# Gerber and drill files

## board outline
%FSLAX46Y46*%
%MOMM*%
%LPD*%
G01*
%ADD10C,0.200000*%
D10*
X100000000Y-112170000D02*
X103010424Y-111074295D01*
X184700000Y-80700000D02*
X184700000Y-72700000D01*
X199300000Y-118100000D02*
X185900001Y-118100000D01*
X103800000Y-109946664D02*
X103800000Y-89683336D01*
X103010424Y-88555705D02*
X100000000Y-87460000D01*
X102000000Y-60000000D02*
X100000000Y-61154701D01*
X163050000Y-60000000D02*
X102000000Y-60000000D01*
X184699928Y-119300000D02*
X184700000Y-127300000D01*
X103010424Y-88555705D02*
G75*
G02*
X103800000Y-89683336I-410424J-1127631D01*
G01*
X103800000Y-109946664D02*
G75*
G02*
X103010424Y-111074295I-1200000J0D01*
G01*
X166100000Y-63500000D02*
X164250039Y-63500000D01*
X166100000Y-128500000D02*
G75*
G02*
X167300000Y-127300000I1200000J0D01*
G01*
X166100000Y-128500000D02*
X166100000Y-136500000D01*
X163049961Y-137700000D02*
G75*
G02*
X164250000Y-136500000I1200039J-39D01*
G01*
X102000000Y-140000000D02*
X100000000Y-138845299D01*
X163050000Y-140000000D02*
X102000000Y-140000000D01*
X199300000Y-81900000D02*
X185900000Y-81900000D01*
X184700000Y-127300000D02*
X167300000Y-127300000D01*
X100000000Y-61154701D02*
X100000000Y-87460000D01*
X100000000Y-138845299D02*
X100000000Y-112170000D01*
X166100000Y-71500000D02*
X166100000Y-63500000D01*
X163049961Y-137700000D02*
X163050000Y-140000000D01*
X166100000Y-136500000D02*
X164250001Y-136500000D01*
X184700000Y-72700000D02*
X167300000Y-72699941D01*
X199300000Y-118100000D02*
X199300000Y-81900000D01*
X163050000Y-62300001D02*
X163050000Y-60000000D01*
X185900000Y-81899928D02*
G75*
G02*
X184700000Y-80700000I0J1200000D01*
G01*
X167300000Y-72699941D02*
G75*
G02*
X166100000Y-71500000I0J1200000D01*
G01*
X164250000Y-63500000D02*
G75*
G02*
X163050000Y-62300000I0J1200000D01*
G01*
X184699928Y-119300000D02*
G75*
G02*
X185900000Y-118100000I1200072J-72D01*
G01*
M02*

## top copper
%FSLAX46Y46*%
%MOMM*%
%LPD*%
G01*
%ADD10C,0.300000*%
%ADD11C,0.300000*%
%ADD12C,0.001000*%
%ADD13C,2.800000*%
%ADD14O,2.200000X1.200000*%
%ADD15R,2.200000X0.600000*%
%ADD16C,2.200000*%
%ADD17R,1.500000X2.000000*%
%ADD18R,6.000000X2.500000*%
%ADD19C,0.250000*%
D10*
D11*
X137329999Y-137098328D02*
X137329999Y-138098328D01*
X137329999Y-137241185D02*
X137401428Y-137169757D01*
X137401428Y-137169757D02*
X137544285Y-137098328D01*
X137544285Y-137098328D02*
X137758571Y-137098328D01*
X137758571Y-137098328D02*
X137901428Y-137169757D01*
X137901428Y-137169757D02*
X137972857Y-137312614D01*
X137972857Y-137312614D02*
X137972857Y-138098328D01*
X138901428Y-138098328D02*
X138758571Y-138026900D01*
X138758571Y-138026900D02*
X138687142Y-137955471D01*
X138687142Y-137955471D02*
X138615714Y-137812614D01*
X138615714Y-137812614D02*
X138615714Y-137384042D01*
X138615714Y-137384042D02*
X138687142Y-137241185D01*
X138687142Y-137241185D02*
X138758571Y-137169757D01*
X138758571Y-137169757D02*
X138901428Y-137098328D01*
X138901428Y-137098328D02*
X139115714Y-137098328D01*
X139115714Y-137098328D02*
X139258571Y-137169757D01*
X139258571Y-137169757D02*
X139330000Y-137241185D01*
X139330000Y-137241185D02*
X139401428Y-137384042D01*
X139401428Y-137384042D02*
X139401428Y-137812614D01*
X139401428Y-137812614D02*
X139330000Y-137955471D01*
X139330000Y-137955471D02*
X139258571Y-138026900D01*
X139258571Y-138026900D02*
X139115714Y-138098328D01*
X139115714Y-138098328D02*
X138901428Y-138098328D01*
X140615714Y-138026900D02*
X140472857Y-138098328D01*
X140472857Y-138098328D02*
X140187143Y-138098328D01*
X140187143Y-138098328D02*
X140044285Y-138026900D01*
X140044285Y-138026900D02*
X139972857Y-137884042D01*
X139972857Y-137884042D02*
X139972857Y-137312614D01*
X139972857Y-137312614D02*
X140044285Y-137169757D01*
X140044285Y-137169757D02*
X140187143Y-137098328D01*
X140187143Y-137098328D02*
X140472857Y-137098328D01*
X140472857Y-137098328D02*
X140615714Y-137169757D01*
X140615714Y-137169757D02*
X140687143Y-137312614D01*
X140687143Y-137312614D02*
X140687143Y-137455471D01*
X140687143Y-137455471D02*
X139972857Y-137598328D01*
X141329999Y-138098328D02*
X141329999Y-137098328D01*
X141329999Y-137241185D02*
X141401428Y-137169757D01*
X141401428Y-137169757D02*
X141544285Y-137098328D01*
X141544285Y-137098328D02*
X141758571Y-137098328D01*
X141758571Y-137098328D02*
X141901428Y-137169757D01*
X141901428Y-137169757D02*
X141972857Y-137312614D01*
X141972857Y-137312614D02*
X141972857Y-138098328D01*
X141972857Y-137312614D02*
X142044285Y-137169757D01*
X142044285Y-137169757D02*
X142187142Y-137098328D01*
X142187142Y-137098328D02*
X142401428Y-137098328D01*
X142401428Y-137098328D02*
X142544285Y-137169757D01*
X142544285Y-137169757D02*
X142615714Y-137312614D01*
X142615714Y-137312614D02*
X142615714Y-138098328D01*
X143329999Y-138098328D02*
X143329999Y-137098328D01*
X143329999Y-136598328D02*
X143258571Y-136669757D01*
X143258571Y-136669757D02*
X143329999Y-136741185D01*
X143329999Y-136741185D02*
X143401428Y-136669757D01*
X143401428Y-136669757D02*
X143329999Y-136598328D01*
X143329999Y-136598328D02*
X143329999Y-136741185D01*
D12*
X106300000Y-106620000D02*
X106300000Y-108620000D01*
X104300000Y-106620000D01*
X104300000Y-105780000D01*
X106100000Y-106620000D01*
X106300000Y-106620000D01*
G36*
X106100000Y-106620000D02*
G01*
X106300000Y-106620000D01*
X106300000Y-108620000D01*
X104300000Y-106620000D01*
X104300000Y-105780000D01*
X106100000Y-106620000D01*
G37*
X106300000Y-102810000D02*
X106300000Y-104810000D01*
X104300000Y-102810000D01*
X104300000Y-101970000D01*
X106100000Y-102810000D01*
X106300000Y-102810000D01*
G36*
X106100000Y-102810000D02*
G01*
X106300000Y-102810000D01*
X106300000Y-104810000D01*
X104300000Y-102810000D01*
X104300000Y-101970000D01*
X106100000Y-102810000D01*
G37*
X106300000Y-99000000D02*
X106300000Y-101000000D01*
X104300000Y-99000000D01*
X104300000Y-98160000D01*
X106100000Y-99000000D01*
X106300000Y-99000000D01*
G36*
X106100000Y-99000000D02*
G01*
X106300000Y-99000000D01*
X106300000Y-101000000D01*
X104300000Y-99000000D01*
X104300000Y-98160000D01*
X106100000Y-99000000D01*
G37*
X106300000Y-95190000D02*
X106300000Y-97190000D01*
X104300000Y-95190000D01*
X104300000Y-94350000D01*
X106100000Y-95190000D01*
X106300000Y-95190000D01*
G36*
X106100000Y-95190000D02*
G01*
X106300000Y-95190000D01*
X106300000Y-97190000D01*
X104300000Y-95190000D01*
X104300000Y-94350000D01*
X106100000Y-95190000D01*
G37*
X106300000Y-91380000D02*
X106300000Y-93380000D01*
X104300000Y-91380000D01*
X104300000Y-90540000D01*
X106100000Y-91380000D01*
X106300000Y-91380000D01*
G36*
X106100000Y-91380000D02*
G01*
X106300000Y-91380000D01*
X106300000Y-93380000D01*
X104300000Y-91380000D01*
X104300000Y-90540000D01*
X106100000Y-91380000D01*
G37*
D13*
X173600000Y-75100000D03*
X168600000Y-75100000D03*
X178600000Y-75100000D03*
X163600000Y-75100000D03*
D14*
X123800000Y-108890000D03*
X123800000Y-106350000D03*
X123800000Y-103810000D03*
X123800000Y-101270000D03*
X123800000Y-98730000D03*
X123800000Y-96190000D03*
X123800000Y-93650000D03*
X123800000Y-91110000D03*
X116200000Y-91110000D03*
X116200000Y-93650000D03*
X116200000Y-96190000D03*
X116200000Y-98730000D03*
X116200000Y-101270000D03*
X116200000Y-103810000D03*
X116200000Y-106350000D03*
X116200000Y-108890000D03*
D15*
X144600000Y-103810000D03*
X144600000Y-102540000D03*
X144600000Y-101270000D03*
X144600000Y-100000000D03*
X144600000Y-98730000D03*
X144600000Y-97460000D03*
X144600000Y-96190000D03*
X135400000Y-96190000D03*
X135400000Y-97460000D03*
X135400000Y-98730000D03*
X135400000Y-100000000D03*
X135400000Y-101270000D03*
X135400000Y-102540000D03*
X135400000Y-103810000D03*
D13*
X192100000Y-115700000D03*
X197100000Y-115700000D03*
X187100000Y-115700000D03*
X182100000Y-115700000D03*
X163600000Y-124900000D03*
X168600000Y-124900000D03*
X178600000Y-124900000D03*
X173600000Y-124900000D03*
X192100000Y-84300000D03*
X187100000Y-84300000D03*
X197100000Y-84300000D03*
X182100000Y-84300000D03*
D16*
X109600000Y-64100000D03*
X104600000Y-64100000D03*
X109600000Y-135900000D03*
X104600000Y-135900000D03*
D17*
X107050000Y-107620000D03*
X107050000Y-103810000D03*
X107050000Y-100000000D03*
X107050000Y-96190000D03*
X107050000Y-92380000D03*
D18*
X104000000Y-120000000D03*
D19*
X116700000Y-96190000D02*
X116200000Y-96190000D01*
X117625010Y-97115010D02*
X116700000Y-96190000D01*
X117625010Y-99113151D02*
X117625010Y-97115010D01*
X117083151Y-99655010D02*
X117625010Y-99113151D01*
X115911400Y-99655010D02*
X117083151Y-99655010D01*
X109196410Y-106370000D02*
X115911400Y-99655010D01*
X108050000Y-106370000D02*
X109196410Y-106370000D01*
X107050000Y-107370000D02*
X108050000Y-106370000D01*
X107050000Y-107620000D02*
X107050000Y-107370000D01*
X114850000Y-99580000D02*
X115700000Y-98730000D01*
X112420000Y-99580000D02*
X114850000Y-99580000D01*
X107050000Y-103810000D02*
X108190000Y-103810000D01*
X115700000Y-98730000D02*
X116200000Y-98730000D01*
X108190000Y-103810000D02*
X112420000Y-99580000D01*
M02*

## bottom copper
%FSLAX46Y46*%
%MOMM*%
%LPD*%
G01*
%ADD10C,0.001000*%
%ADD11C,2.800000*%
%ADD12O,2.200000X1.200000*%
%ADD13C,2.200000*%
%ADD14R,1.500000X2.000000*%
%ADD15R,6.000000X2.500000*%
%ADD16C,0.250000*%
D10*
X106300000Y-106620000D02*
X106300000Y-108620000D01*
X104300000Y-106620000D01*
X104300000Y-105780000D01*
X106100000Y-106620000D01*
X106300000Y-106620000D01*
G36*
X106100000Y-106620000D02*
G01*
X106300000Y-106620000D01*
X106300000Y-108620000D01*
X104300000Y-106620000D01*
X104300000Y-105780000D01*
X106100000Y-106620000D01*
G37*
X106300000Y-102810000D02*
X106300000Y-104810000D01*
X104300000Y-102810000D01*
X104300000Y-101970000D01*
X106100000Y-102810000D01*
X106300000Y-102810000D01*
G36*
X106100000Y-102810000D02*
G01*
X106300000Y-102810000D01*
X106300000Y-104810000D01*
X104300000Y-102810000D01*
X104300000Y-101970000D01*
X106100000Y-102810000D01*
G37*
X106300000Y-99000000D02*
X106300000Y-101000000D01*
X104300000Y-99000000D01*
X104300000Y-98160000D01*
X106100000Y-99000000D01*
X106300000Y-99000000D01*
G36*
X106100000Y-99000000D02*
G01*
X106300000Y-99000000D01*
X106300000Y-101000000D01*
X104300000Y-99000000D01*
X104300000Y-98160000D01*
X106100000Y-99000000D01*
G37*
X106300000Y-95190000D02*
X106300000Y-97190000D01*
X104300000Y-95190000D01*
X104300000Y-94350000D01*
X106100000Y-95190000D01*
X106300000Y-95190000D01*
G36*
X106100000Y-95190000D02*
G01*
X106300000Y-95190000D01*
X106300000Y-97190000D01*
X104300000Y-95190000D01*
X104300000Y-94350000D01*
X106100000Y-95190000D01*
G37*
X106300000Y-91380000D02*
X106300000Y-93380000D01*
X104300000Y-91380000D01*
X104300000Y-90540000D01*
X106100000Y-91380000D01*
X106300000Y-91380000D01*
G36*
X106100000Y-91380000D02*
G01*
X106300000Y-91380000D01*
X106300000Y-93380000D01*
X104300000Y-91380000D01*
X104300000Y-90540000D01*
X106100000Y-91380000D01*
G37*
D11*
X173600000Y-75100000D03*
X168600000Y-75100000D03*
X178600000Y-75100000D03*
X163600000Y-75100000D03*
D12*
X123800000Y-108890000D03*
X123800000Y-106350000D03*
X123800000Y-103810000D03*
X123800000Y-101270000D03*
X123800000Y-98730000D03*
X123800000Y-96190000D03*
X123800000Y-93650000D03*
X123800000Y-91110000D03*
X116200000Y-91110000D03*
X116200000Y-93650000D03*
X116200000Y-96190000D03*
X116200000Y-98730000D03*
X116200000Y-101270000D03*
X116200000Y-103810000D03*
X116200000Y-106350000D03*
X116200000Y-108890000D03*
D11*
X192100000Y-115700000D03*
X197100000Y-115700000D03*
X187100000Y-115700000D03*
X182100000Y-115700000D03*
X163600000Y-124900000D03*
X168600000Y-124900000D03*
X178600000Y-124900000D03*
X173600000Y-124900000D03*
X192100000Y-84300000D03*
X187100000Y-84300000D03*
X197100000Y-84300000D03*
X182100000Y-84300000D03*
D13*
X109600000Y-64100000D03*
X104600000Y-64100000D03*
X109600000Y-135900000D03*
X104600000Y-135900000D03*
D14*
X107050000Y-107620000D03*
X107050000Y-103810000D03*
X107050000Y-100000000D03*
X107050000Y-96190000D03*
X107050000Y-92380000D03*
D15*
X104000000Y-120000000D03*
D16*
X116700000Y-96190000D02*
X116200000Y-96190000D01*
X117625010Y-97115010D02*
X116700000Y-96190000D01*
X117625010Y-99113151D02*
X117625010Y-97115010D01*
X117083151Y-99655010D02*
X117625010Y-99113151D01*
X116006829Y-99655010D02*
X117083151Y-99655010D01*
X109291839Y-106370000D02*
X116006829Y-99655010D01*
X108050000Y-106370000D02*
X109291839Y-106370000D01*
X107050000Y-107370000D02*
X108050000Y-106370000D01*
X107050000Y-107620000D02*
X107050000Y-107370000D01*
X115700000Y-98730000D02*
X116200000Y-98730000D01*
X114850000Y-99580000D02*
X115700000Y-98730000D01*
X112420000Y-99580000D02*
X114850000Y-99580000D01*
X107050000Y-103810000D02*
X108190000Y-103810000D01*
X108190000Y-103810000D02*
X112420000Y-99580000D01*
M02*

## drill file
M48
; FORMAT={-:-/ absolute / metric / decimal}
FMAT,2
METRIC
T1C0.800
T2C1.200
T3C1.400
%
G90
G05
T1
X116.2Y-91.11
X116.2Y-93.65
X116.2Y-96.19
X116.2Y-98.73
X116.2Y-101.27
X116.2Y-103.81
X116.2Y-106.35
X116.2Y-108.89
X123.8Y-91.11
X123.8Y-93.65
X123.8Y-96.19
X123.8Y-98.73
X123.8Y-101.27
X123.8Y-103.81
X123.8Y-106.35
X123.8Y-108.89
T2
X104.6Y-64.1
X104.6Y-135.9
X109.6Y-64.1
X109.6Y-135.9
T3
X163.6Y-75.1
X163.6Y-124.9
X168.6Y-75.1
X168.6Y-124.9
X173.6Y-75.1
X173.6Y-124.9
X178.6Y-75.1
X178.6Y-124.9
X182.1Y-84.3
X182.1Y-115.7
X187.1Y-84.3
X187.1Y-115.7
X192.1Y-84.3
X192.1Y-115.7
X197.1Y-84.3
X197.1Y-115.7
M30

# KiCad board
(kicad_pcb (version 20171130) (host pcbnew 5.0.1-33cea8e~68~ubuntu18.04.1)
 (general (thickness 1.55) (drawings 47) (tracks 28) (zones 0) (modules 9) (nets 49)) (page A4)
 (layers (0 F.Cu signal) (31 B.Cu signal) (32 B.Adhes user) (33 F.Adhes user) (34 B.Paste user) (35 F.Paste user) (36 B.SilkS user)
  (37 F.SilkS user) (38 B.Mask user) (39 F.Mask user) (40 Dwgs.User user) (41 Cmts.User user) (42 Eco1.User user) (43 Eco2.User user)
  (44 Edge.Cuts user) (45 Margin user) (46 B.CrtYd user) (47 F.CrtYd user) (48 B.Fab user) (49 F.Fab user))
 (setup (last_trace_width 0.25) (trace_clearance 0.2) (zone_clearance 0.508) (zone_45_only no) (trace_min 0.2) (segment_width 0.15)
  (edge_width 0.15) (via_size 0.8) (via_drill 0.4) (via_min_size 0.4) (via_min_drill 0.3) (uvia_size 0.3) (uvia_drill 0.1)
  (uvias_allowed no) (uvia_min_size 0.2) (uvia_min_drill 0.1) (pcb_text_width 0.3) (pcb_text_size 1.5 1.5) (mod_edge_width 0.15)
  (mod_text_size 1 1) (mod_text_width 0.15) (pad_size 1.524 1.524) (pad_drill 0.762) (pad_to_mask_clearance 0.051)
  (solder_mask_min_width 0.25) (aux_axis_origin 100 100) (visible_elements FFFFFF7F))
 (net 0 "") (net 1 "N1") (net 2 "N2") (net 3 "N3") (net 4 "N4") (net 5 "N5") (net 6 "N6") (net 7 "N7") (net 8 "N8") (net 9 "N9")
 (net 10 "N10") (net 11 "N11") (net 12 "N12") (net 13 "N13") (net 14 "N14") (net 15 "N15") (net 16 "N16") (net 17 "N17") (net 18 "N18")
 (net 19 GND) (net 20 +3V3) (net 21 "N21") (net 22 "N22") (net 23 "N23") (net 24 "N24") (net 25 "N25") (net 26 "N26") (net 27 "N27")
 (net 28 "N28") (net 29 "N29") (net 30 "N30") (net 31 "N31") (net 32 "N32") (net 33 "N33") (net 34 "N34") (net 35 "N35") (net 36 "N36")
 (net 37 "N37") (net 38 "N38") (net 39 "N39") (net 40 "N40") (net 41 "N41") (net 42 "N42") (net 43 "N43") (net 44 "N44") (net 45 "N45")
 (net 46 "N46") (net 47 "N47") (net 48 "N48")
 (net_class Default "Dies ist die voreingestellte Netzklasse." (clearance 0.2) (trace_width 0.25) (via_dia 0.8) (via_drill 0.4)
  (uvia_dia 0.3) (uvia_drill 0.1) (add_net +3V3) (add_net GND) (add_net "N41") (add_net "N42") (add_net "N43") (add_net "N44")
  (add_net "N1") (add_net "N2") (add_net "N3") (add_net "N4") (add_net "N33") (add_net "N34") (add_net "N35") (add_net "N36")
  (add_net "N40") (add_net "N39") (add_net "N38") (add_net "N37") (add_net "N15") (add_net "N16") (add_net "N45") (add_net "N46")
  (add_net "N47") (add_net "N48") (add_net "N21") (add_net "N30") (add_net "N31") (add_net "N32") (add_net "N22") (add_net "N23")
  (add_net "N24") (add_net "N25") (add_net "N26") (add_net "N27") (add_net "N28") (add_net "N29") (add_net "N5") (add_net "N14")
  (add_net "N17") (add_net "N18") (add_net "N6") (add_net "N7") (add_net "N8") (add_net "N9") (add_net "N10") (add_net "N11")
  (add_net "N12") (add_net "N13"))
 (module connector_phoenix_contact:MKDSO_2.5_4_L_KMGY (layer F.Cu) (at 171.1 75.1 270)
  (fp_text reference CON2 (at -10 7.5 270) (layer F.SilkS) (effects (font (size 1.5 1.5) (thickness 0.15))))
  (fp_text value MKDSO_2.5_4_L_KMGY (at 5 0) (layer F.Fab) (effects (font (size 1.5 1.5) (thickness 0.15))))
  (pad 1 thru_hole circle (at 0 -2.5 270) (size 2.8 2.8) (drill 1.4) (layers *.Cu *.Mask) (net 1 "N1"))
  (pad 2 thru_hole circle (at 0 2.5 270) (size 2.8 2.8) (drill 1.4) (layers *.Cu *.Mask) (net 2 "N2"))
  (pad 3 thru_hole circle (at 0 -7.5 270) (size 2.8 2.8) (drill 1.4) (layers *.Cu *.Mask) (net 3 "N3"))
  (pad 4 thru_hole circle (at 0 7.5 270) (size 2.8 2.8) (drill 1.4) (layers *.Cu *.Mask) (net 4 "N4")))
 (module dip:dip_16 (layer F.Cu) (at 120 100 90)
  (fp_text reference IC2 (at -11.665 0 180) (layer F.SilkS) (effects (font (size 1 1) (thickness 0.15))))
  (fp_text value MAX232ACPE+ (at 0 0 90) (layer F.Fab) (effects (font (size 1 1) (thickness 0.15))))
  (pad 1 thru_hole oval (at -8.89 3.8 90) (size 1.2 2.2) (drill 0.8) (layers *.Cu *.Mask) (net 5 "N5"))
  (pad 2 thru_hole oval (at -6.35 3.8 90) (size 1.2 2.2) (drill 0.8) (layers *.Cu *.Mask) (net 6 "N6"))
  (pad 3 thru_hole oval (at -3.81 3.8 90) (size 1.2 2.2) (drill 0.8) (layers *.Cu *.Mask) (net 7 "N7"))
  (pad 4 thru_hole oval (at -1.27 3.8 90) (size 1.2 2.2) (drill 0.8) (layers *.Cu *.Mask) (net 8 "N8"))
  (pad 5 thru_hole oval (at 1.27 3.8 90) (size 1.2 2.2) (drill 0.8) (layers *.Cu *.Mask) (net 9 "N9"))
  (pad 6 thru_hole oval (at 3.81 3.8 90) (size 1.2 2.2) (drill 0.8) (layers *.Cu *.Mask) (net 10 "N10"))
  (pad 7 thru_hole oval (at 6.35 3.8 90) (size 1.2 2.2) (drill 0.8) (layers *.Cu *.Mask) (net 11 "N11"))
  (pad 8 thru_hole oval (at 8.89 3.8 90) (size 1.2 2.2) (drill 0.8) (layers *.Cu *.Mask) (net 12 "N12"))
  (pad 9 thru_hole oval (at 8.89 -3.8 90) (size 1.2 2.2) (drill 0.8) (layers *.Cu *.Mask) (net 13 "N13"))
  (pad 10 thru_hole oval (at 6.35 -3.8 90) (size 1.2 2.2) (drill 0.8) (layers *.Cu *.Mask) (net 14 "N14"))
  (pad 11 thru_hole oval (at 3.81 -3.8 90) (size 1.2 2.2) (drill 0.8) (layers *.Cu *.Mask) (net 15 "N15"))
  (pad 12 thru_hole oval (at 1.27 -3.8 90) (size 1.2 2.2) (drill 0.8) (layers *.Cu *.Mask) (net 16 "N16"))
  (pad 13 thru_hole oval (at -1.27 -3.8 90) (size 1.2 2.2) (drill 0.8) (layers *.Cu *.Mask) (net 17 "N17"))
  (pad 14 thru_hole oval (at -3.81 -3.8 90) (size 1.2 2.2) (drill 0.8) (layers *.Cu *.Mask) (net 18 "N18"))
  (pad 15 thru_hole oval (at -6.35 -3.8 90) (size 1.2 2.2) (drill 0.8) (layers *.Cu *.Mask) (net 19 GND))
  (pad 16 thru_hole oval (at -8.89 -3.8 90) (size 1.2 2.2) (drill 0.8) (layers *.Cu *.Mask) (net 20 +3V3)))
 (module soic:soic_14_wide (layer F.Cu) (at 140 100 90)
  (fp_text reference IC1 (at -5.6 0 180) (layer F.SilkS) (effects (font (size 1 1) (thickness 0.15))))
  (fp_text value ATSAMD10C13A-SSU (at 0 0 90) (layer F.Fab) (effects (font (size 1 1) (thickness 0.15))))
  (pad 1 smd rect (at -3.81 4.6 90) (size 0.6 2.2) (layers F.Cu F.Paste F.Mask) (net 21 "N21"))
  (pad 2 smd rect (at -2.54 4.6 90) (size 0.6 2.2) (layers F.Cu F.Paste F.Mask) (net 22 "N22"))
  (pad 3 smd rect (at -1.27 4.6 90) (size 0.6 2.2) (layers F.Cu F.Paste F.Mask) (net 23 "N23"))
  (pad 4 smd rect (at 0 4.6 90) (size 0.6 2.2) (layers F.Cu F.Paste F.Mask) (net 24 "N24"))
  (pad 5 smd rect (at 1.27 4.6 90) (size 0.6 2.2) (layers F.Cu F.Paste F.Mask) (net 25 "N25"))
  (pad 6 smd rect (at 2.54 4.6 90) (size 0.6 2.2) (layers F.Cu F.Paste F.Mask) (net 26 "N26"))
  (pad 7 smd rect (at 3.81 4.6 90) (size 0.6 2.2) (layers F.Cu F.Paste F.Mask) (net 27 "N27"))
  (pad 8 smd rect (at 3.81 -4.6 90) (size 0.6 2.2) (layers F.Cu F.Paste F.Mask) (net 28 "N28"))
  (pad 9 smd rect (at 2.54 -4.6 90) (size 0.6 2.2) (layers F.Cu F.Paste F.Mask) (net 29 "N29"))
  (pad 10 smd rect (at 1.27 -4.6 90) (size 0.6 2.2) (layers F.Cu F.Paste F.Mask) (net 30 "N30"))
  (pad 11 smd rect (at 0 -4.6 90) (size 0.6 2.2) (layers F.Cu F.Paste F.Mask))
  (pad 12 smd rect (at -1.27 -4.6 90) (size 0.6 2.2) (layers F.Cu F.Paste F.Mask))
  (pad 13 smd rect (at -2.54 -4.6 90) (size 0.6 2.2) (layers F.Cu F.Paste F.Mask) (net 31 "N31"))
  (pad 14 smd rect (at -3.81 -4.6 90) (size 0.6 2.2) (layers F.Cu F.Paste F.Mask) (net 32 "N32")))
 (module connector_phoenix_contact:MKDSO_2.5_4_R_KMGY (layer F.Cu) (at 189.6 115.7 270)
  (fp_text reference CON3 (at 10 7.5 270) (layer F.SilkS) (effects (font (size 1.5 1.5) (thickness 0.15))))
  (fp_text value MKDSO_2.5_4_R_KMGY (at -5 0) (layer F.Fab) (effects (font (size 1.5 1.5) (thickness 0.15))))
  (pad 1 thru_hole circle (at 0 -2.5 270) (size 2.8 2.8) (drill 1.4) (layers *.Cu *.Mask) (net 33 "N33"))
  (pad 2 thru_hole circle (at 0 -7.5 270) (size 2.8 2.8) (drill 1.4) (layers *.Cu *.Mask) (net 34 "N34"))
  (pad 3 thru_hole circle (at 0 2.5 270) (size 2.8 2.8) (drill 1.4) (layers *.Cu *.Mask) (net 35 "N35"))
  (pad 4 thru_hole circle (at 0 7.5 270) (size 2.8 2.8) (drill 1.4) (layers *.Cu *.Mask) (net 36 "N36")))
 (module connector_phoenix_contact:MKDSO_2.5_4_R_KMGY (layer F.Cu) (at 171.1 124.9 270)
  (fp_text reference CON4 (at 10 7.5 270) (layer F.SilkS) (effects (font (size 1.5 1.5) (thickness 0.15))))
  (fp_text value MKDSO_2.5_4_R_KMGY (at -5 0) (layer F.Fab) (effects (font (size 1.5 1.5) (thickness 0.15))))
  (pad 4 thru_hole circle (at 0 7.5 270) (size 2.8 2.8) (drill 1.4) (layers *.Cu *.Mask) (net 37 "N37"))
  (pad 3 thru_hole circle (at 0 2.5 270) (size 2.8 2.8) (drill 1.4) (layers *.Cu *.Mask) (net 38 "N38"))
  (pad 2 thru_hole circle (at 0 -7.5 270) (size 2.8 2.8) (drill 1.4) (layers *.Cu *.Mask) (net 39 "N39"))
  (pad 1 thru_hole circle (at 0 -2.5 270) (size 2.8 2.8) (drill 1.4) (layers *.Cu *.Mask) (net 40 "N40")))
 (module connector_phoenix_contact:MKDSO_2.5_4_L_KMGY (layer F.Cu) (at 189.6 84.3 270)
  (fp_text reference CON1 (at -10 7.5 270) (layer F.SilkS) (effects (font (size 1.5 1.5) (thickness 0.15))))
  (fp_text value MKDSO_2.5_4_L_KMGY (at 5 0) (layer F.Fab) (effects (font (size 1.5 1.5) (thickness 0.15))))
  (pad 1 thru_hole circle (at 0 -2.5 270) (size 2.8 2.8) (drill 1.4) (layers *.Cu *.Mask) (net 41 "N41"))
  (pad 2 thru_hole circle (at 0 2.5 270) (size 2.8 2.8) (drill 1.4) (layers *.Cu *.Mask) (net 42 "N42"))
  (pad 3 thru_hole circle (at 0 -7.5 270) (size 2.8 2.8) (drill 1.4) (layers *.Cu *.Mask) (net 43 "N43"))
  (pad 4 thru_hole circle (at 0 7.5 270) (size 2.8 2.8) (drill 1.4) (layers *.Cu *.Mask) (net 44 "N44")))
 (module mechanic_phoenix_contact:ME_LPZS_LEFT (layer F.Cu) (at 107.1 64.1)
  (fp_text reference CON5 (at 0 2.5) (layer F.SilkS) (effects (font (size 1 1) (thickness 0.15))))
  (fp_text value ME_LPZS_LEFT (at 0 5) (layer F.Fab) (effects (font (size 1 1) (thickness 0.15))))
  (pad "" thru_hole circle (at 2.5 0) (size 2.2 2.2) (drill 1.2) (layers *.Cu *.Mask))
  (pad "" thru_hole circle (at -2.5 0) (size 2.2 2.2) (drill 1.2) (layers *.Cu *.Mask)))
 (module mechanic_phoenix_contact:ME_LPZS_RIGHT (layer F.Cu) (at 107.1 135.9)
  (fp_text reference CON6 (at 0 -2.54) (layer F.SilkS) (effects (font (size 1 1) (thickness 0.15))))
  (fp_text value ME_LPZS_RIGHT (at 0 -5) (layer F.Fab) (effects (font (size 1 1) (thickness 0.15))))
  (pad "" thru_hole circle (at 2.5 0) (size 2.2 2.2) (drill 1.2) (layers *.Cu *.Mask))
  (pad "" thru_hole circle (at -2.5 0) (size 2.2 2.2) (drill 1.2) (layers *.Cu *.Mask)))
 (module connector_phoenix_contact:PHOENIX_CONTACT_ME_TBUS (layer F.Cu) (at 103.8 100 270)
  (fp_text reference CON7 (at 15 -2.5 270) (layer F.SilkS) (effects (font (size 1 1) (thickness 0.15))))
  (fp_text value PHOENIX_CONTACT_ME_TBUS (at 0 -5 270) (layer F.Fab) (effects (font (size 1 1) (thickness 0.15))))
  (fp_poly (pts (xy 6.62 -2.5) (xy 8.62 -2.5) (xy 6.62 -0.5) (xy 5.78 -0.5) (xy 6.62 -2.3)) (layer B.Cu) (width 0.001))
  (fp_poly (pts (xy 2.81 -2.5) (xy 4.81 -2.5) (xy 2.81 -0.5) (xy 1.97 -0.5) (xy 2.81 -2.3)) (layer B.Cu) (width 0.001))
  (fp_poly (pts (xy -1 -2.5) (xy 1 -2.5) (xy -1 -0.5) (xy -1.84 -0.5) (xy -1 -2.3)) (layer B.Cu) (width 0.001))
  (fp_poly (pts (xy -4.81 -2.5) (xy -2.81 -2.5) (xy -4.81 -0.5) (xy -5.65 -0.5) (xy -4.81 -2.3)) (layer B.Cu) (width 0.001))
  (fp_poly (pts (xy 6.62 -2.5) (xy 8.62 -2.5) (xy 6.62 -0.5) (xy 5.78 -0.5) (xy 6.62 -2.3)) (layer F.Cu) (width 0.001))
  (fp_poly (pts (xy 2.81 -2.5) (xy 4.81 -2.5) (xy 2.81 -0.5) (xy 1.97 -0.5) (xy 2.81 -2.3)) (layer F.Cu) (width 0.001))
  (fp_poly (pts (xy -1 -2.5) (xy 1 -2.5) (xy -1 -0.5) (xy -1.84 -0.5) (xy -1 -2.3)) (layer F.Cu) (width 0.001))
  (fp_poly (pts (xy -4.81 -2.5) (xy -2.81 -2.5) (xy -4.81 -0.5) (xy -5.65 -0.5) (xy -4.81 -2.3)) (layer F.Cu) (width 0.001))
  (fp_poly (pts (xy -8.62 -2.5) (xy -6.62 -2.5) (xy -8.62 -0.5) (xy -9.46 -0.5) (xy -8.62 -2.3)) (layer F.Cu) (width 0.001))
  (fp_poly (pts (xy -8.62 -2.5) (xy -6.62 -2.5) (xy -8.62 -0.5) (xy -9.46 -0.5) (xy -8.62 -2.3)) (layer B.Cu) (width 0.001))
  (pad 1 connect rect (at 7.62 -3.25 270) (size 2 1.5) (layers F.Cu F.Mask) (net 15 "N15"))
  (pad 1 connect rect (at 7.62 -3.25 270) (size 2 1.5) (layers B.Cu B.Mask) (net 15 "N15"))
  (pad 2 connect rect (at 3.81 -3.25 270) (size 2 1.5) (layers F.Cu F.Mask) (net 16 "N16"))
  (pad 2 connect rect (at 3.81 -3.25 270) (size 2 1.5) (layers B.Cu B.Mask) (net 16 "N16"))
  (pad 3 connect rect (at 0 -3.25 270) (size 2 1.5) (layers F.Cu F.Mask) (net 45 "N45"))
  (pad 3 connect rect (at 0 -3.25 270) (size 2 1.5) (layers B.Cu B.Mask) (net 45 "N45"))
  (pad 4 connect rect (at -3.81 -3.25 270) (size 2 1.5) (layers F.Cu F.Mask) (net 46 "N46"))
  (pad 4 connect rect (at -3.81 -3.25 270) (size 2 1.5) (layers B.Cu B.Mask) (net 46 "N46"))
  (pad 5 connect rect (at -7.62 -3.25 270) (size 2 1.5) (layers F.Cu F.Mask) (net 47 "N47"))
  (pad 5 connect rect (at -7.62 -3.25 270) (size 2 1.5) (layers B.Cu B.Mask) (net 47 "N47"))
  (pad 6 connect rect (at 20 -0.2 270) (size 2.5 6) (layers F.Cu F.Mask) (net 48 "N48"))
  (pad 6 connect rect (at 20 -0.2 270) (size 2.5 6) (layers B.Cu B.Mask) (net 48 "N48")))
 (gr_line (start 100 112.17) (end 103.010424 111.074295) (layer Edge.Cuts) (width 0.2))
 (gr_line (start 184.7 80.7) (end 184.7 72.7) (layer Edge.Cuts) (width 0.2))
 (gr_line (start 199.3 118.1) (end 185.900001 118.1) (layer Edge.Cuts) (width 0.2))
 (gr_line (start 103.8 109.946664) (end 103.8 89.683336) (layer Edge.Cuts) (width 0.2))
 (gr_line (start 103.010424 88.555705) (end 100 87.46) (layer Edge.Cuts) (width 0.2))
 (gr_line (start 102 60) (end 100 61.154701) (layer Edge.Cuts) (width 0.2))
 (gr_line (start 163.05 60) (end 102 60) (layer Edge.Cuts) (width 0.2))
 (gr_line (start 184.699928 119.3) (end 184.7 127.3) (layer Edge.Cuts) (width 0.2))
 (gr_arc (start 102.6 89.683336) (end 103.8 89.683336) (angle -70.00001527) (layer Edge.Cuts) (width 0.2))
 (gr_arc (start 102.6 109.946664) (end 103.010424 111.074295) (angle -70.00000108) (layer Edge.Cuts) (width 0.2))
 (gr_line (start 166.1 63.5) (end 164.250039 63.5) (layer Edge.Cuts) (width 0.2))
 (gr_arc (start 167.3 128.5) (end 167.3 127.3) (angle -89.99999993) (layer Edge.Cuts) (width 0.2))
 (gr_line (start 166.1 128.5) (end 166.1 136.5) (layer Edge.Cuts) (width 0.2))
 (gr_arc (start 164.25 137.700039) (end 164.25 136.5) (angle -89.99811922) (layer Edge.Cuts) (width 0.2))
 (gr_line (start 102 140) (end 100 138.845299) (layer Edge.Cuts) (width 0.2))
 (gr_line (start 163.05 140) (end 102 140) (layer Edge.Cuts) (width 0.2))
 (gr_line (start 199.3 81.9) (end 185.9 81.9) (layer Edge.Cuts) (width 0.2))
 (gr_line (start 184.7 127.3) (end 167.3 127.3) (layer Edge.Cuts) (width 0.2))
 (gr_line (start 100 61.154701) (end 100 87.46) (layer Edge.Cuts) (width 0.2))
 (gr_line (start 100 138.845299) (end 100 112.17) (layer Edge.Cuts) (width 0.2))
 (gr_line (start 166.1 71.5) (end 166.1 63.5) (layer Edge.Cuts) (width 0.2))
 (gr_line (start 163.049961 137.7) (end 163.05 140) (layer Edge.Cuts) (width 0.2))
 (gr_line (start 166.1 136.5) (end 164.250001 136.5) (layer Edge.Cuts) (width 0.2))
 (gr_line (start 184.7 72.7) (end 167.3 72.699941) (layer Edge.Cuts) (width 0.2))
 (gr_line (start 199.3 118.1) (end 199.3 81.9) (layer Edge.Cuts) (width 0.2))
 (gr_line (start 163.05 62.300001) (end 163.05 60) (layer Edge.Cuts) (width 0.2))
 (gr_arc (start 185.9 80.699928) (end 184.7 80.7) (angle -89.99657278) (layer Edge.Cuts) (width 0.2))
 (gr_arc (start 167.3 71.499941) (end 166.1 71.5) (angle -89.99717399) (layer Edge.Cuts) (width 0.2))
 (gr_arc (start 164.25 62.3) (end 163.05 62.3) (angle -89.99999997) (layer Edge.Cuts) (width 0.2))
 (gr_arc (start 185.9 119.300072) (end 185.9 118.1) (angle -89.99657278) (layer Edge.Cuts) (width 0.2))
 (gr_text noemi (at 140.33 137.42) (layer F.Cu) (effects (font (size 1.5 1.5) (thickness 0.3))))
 (segment (start 116.7 96.19) (end 116.2 96.19) (width 0.25) (layer F.Cu) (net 15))
 (segment (start 117.62501 97.11501) (end 116.7 96.19) (width 0.25) (layer F.Cu) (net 15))
 (segment (start 117.62501 99.113151) (end 117.62501 97.11501) (width 0.25) (layer F.Cu) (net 15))
 (segment (start 117.083151 99.65501) (end 117.62501 99.113151) (width 0.25) (layer F.Cu) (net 15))
 (segment (start 115.9114 99.65501) (end 117.083151 99.65501) (width 0.25) (layer F.Cu) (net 15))
 (segment (start 109.19641 106.37) (end 115.9114 99.65501) (width 0.25) (layer F.Cu) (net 15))
 (segment (start 108.05 106.37) (end 109.19641 106.37) (width 0.25) (layer F.Cu) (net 15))
 (segment (start 107.05 107.37) (end 108.05 106.37) (width 0.25) (layer F.Cu) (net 15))
 (segment (start 107.05 107.62) (end 107.05 107.37) (width 0.25) (layer F.Cu) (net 15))
 (segment (start 116.7 96.19) (end 116.2 96.19) (width 0.25) (layer B.Cu) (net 15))
 (segment (start 117.62501 97.11501) (end 116.7 96.19) (width 0.25) (layer B.Cu) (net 15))
 (segment (start 117.62501 99.113151) (end 117.62501 97.11501) (width 0.25) (layer B.Cu) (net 15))
 (segment (start 117.083151 99.65501) (end 117.62501 99.113151) (width 0.25) (layer B.Cu) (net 15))
 (segment (start 116.006829 99.65501) (end 117.083151 99.65501) (width 0.25) (layer B.Cu) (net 15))
 (segment (start 109.291839 106.37) (end 116.006829 99.65501) (width 0.25) (layer B.Cu) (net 15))
 (segment (start 108.05 106.37) (end 109.291839 106.37) (width 0.25) (layer B.Cu) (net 15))
 (segment (start 107.05 107.37) (end 108.05 106.37) (width 0.25) (layer B.Cu) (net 15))
 (segment (start 107.05 107.62) (end 107.05 107.37) (width 0.25) (layer B.Cu) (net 15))
 (segment (start 115.7 98.73) (end 116.2 98.73) (width 0.25) (layer B.Cu) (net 16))
 (segment (start 114.85 99.58) (end 115.7 98.73) (width 0.25) (layer B.Cu) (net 16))
 (segment (start 112.42 99.58) (end 114.85 99.58) (width 0.25) (layer B.Cu) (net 16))
 (segment (start 107.05 103.81) (end 108.19 103.81) (width 0.25) (layer B.Cu) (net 16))
 (segment (start 108.19 103.81) (end 112.42 99.58) (width 0.25) (layer B.Cu) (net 16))
 (segment (start 114.85 99.58) (end 115.7 98.73) (width 0.25) (layer F.Cu) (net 16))
 (segment (start 112.42 99.58) (end 114.85 99.58) (width 0.25) (layer F.Cu) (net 16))
 (segment (start 107.05 103.81) (end 108.19 103.81) (width 0.25) (layer F.Cu) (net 16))
 (segment (start 115.7 98.73) (end 116.2 98.73) (width 0.25) (layer F.Cu) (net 16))
 (segment (start 108.19 103.81) (end 112.42 99.58) (width 0.25) (layer F.Cu) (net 16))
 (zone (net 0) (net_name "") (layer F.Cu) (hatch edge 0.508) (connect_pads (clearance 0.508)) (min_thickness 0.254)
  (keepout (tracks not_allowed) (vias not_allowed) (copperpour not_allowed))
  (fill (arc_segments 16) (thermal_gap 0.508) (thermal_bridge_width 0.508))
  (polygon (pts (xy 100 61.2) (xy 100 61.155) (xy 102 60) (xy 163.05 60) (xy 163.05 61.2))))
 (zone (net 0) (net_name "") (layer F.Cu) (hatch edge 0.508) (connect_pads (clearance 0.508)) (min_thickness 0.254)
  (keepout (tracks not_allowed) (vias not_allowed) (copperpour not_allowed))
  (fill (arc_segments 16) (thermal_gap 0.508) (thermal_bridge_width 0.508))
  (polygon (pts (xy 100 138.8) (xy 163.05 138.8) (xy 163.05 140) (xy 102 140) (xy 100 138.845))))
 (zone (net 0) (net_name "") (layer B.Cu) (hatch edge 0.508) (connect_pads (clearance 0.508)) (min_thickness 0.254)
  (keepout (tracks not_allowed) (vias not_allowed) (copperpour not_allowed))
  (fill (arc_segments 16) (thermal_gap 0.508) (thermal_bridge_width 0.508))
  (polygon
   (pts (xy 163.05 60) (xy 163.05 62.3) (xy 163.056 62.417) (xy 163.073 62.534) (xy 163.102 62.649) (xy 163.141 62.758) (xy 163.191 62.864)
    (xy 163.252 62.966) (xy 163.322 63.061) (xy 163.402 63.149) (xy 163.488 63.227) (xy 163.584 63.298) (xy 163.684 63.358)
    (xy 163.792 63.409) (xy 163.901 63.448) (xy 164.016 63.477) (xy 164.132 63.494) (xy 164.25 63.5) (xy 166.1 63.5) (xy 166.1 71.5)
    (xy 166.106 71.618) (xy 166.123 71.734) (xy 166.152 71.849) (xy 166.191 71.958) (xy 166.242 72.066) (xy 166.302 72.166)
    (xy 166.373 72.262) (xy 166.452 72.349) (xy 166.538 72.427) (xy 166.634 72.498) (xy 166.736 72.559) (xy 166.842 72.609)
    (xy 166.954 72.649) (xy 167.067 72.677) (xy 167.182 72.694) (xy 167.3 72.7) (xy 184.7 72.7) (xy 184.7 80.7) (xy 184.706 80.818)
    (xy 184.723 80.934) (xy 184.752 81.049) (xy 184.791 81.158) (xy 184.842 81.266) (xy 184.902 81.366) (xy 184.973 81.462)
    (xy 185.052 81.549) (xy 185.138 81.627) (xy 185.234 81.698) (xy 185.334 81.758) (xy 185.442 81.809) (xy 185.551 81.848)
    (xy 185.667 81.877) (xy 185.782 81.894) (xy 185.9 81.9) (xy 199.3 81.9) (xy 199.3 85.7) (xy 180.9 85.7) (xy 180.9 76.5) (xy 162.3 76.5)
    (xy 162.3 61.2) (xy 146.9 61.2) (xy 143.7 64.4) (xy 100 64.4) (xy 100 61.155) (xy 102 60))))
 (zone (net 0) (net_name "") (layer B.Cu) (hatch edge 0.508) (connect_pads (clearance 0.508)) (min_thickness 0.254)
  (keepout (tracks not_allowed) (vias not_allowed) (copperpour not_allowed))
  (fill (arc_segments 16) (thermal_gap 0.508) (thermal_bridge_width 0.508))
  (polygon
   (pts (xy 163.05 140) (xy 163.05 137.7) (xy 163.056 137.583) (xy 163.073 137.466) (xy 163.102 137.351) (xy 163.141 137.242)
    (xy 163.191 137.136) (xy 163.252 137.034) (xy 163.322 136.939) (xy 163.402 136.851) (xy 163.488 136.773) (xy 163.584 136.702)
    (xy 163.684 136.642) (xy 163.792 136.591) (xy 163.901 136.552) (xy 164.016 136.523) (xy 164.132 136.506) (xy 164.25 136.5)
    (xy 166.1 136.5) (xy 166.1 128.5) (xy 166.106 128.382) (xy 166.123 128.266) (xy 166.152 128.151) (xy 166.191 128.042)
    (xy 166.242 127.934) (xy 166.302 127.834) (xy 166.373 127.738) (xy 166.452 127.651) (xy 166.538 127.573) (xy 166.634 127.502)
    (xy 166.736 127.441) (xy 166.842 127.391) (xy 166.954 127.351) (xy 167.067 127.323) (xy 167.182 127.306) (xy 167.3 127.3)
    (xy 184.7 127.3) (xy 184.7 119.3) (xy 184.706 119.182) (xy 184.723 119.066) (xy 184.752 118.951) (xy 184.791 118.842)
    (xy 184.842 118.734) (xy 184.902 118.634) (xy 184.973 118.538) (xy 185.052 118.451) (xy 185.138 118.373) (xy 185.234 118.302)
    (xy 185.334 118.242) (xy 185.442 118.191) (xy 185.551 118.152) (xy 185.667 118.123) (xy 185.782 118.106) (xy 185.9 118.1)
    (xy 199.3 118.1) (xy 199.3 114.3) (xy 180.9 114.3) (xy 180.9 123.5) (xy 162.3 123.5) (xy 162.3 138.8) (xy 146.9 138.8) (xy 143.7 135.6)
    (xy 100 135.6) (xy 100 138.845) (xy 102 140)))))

